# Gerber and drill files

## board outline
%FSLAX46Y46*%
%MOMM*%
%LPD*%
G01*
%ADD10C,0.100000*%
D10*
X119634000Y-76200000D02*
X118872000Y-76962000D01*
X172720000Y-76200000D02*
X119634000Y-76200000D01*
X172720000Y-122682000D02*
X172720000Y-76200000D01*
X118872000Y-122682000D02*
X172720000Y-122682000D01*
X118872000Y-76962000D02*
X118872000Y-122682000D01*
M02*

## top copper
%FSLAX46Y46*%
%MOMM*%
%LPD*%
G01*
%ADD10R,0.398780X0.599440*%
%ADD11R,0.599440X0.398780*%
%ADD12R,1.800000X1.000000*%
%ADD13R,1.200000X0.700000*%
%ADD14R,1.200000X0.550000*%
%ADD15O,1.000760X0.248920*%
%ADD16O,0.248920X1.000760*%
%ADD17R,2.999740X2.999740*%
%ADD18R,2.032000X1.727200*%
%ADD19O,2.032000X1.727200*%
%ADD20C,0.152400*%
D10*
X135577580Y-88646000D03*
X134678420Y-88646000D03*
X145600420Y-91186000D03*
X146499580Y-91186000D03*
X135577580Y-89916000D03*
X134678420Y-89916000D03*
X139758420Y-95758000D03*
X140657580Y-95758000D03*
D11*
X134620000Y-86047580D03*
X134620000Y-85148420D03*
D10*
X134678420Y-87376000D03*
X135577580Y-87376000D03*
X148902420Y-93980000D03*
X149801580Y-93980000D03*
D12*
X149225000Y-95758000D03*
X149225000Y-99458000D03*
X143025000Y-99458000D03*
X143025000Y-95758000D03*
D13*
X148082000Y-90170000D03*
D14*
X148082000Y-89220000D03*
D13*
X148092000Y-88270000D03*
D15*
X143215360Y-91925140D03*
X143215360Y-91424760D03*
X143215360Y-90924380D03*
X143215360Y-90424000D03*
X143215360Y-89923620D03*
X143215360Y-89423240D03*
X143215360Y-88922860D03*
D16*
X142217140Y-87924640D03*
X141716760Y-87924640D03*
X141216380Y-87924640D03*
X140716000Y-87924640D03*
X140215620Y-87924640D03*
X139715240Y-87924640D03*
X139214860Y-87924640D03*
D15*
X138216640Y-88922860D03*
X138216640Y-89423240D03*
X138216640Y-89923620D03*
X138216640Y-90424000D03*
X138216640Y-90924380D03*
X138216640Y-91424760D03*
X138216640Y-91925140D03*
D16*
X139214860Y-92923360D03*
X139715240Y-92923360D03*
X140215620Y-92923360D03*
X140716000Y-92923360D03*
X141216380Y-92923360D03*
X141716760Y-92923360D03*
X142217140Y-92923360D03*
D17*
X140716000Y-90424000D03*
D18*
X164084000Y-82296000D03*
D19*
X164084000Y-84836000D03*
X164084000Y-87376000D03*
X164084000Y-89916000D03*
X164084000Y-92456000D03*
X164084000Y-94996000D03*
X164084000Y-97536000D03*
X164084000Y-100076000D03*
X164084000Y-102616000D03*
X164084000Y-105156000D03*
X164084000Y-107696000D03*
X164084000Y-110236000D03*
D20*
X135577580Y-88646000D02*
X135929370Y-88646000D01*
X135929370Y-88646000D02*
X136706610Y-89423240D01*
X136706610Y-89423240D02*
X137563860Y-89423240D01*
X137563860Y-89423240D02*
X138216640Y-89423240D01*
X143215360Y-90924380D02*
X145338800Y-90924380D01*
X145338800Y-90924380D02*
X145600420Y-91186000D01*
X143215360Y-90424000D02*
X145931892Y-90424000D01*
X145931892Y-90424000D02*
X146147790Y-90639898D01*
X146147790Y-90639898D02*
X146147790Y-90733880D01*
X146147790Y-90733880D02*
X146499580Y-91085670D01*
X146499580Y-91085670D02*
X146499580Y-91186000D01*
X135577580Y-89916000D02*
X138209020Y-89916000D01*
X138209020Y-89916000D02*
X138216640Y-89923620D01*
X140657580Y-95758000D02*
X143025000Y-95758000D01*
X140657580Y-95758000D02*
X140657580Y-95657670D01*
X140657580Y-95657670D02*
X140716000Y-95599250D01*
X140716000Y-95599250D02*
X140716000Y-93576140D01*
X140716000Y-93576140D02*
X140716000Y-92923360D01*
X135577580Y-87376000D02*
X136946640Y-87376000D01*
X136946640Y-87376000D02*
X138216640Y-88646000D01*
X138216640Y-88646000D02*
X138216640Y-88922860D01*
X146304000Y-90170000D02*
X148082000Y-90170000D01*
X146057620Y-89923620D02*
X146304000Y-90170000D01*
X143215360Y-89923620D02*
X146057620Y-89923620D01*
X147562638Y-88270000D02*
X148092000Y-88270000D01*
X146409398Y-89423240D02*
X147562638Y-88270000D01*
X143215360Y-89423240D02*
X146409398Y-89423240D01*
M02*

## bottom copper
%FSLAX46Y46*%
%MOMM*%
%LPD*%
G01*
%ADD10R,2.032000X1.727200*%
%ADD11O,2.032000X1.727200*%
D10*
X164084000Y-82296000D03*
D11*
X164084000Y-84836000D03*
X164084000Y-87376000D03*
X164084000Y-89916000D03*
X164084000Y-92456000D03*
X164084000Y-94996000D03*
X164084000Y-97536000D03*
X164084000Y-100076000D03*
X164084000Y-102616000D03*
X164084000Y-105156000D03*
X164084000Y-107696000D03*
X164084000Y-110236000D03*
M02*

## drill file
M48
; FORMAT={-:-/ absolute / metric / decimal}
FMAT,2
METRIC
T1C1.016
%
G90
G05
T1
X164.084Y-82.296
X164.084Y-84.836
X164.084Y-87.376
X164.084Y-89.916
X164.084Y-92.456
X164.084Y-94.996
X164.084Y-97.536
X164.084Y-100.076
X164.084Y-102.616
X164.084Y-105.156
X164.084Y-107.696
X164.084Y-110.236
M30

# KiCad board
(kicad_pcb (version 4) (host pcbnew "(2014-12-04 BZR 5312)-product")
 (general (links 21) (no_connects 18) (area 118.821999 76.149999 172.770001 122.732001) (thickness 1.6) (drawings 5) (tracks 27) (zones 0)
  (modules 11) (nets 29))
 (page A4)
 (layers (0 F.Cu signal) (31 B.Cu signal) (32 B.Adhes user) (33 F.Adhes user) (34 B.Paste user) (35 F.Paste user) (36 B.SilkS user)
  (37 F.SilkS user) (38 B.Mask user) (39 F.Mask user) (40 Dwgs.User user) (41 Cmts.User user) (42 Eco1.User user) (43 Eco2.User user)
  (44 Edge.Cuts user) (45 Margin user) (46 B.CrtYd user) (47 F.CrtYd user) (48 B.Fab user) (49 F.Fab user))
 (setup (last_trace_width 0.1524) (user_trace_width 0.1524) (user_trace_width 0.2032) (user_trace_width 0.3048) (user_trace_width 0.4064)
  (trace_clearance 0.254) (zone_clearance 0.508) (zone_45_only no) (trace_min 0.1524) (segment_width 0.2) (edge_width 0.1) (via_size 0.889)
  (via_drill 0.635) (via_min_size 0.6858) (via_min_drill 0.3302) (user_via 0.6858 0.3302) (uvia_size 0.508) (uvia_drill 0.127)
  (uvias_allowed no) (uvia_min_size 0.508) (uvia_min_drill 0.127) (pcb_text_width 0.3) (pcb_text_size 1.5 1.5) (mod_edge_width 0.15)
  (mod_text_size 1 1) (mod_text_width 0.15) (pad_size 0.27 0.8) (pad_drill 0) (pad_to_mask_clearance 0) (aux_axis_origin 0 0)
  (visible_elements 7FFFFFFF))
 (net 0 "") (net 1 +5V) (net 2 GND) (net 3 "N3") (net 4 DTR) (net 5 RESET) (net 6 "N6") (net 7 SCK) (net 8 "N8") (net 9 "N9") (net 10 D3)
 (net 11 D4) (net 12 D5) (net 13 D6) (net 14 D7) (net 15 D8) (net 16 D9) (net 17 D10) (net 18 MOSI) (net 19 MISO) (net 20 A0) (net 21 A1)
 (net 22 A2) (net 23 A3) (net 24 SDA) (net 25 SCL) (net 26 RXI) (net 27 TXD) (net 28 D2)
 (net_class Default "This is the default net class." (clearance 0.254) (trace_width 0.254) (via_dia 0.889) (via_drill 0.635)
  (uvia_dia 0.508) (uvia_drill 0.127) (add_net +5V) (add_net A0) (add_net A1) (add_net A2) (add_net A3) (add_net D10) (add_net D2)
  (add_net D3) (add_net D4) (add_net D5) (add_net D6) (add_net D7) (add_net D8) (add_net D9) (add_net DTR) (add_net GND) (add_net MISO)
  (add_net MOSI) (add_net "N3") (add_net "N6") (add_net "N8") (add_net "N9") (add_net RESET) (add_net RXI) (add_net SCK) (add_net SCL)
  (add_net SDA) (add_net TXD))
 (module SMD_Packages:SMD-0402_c (layer F.Cu) (at 135.128 88.646 180)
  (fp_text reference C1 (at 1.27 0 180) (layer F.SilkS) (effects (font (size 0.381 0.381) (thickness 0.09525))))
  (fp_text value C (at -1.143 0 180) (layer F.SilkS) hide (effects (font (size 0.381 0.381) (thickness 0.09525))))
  (pad 1 smd rect (at -0.44958 0 180) (size 0.39878 0.59944) (layers F.Cu F.Paste F.Mask) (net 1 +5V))
  (pad 2 smd rect (at 0.44958 0 180) (size 0.39878 0.59944) (layers F.Cu F.Paste F.Mask) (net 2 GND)))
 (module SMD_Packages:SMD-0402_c (layer F.Cu) (at 146.05 91.186)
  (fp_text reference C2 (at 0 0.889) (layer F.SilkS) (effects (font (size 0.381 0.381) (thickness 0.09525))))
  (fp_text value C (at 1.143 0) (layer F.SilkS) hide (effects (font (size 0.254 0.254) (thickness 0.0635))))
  (pad 1 smd rect (at -0.44958 0) (size 0.39878 0.59944) (layers F.Cu F.Paste F.Mask) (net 1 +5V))
  (pad 2 smd rect (at 0.44958 0) (size 0.39878 0.59944) (layers F.Cu F.Paste F.Mask) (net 2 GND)))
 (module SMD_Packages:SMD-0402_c (layer F.Cu) (at 135.128 89.916 180)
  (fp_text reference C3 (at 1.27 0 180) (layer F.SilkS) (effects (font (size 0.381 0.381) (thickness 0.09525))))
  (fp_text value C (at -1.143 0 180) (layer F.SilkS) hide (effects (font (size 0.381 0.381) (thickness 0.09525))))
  (pad 1 smd rect (at -0.44958 0 180) (size 0.39878 0.59944) (layers F.Cu F.Paste F.Mask) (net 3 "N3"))
  (pad 2 smd rect (at 0.44958 0 180) (size 0.39878 0.59944) (layers F.Cu F.Paste F.Mask) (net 2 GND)))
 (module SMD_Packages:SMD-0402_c (layer F.Cu) (at 140.208 95.758)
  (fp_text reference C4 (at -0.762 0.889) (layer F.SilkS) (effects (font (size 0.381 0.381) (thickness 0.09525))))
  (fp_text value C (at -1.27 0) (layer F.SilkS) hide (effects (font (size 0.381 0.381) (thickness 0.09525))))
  (pad 1 smd rect (at -0.44958 0) (size 0.39878 0.59944) (layers F.Cu F.Paste F.Mask) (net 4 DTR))
  (pad 2 smd rect (at 0.44958 0) (size 0.39878 0.59944) (layers F.Cu F.Paste F.Mask) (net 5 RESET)))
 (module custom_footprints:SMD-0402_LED (layer F.Cu) (at 134.62 85.598 90)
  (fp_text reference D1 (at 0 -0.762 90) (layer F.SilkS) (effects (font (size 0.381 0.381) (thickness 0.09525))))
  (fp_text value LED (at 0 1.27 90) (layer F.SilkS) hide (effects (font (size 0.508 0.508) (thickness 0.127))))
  (pad 1 smd rect (at -0.44958 0 90) (size 0.39878 0.59944) (layers F.Cu F.Paste F.Mask) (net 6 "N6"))
  (pad 2 smd rect (at 0.44958 0 90) (size 0.39878 0.59944) (layers F.Cu F.Paste F.Mask) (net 2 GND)))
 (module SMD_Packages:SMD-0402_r (layer F.Cu) (at 135.128 87.376)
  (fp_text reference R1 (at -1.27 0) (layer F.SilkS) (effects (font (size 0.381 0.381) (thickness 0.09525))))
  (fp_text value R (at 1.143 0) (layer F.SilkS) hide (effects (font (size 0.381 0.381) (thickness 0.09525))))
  (pad 1 smd rect (at -0.44958 0) (size 0.39878 0.59944) (layers F.Cu F.Paste F.Mask) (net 6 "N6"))
  (pad 2 smd rect (at 0.44958 0) (size 0.39878 0.59944) (layers F.Cu F.Paste F.Mask) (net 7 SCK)))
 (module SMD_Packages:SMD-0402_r (layer F.Cu) (at 149.352 93.98)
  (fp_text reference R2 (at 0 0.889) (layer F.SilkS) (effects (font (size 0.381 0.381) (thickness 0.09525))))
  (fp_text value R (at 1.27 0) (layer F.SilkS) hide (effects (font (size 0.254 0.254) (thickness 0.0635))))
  (pad 1 smd rect (at -0.44958 0) (size 0.39878 0.59944) (layers F.Cu F.Paste F.Mask) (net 1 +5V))
  (pad 2 smd rect (at 0.44958 0) (size 0.39878 0.59944) (layers F.Cu F.Paste F.Mask) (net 5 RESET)))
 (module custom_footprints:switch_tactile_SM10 (layer F.Cu) (at 149.225 95.758 180) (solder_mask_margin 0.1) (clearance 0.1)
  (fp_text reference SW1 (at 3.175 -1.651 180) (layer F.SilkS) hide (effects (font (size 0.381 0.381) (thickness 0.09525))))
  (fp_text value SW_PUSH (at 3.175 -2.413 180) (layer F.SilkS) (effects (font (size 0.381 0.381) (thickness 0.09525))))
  (pad 1 smd rect (at 0 0 180) (size 1.8 1) (layers F.Cu F.Paste F.Mask) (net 5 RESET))
  (pad 2 smd rect (at 0 -3.7 180) (size 1.8 1) (layers F.Cu F.Paste F.Mask) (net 2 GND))
  (pad 2 smd rect (at 6.2 -3.7 180) (size 1.8 1) (layers F.Cu F.Paste F.Mask) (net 2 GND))
  (pad 1 smd rect (at 6.2 0 180) (size 1.8 1) (layers F.Cu F.Paste F.Mask) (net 5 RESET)))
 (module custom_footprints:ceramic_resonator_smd (layer F.Cu) (at 148.082 90.17 90) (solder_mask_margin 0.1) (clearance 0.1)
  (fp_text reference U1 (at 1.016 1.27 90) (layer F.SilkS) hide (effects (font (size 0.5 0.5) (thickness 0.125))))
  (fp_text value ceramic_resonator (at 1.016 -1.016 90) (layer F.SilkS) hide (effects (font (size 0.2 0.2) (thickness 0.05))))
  (pad 1 smd rect (at 0 0 90) (size 0.7 1.2) (layers F.Cu F.Paste F.Mask) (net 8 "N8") (solder_mask_margin 0.1) (clearance 0.1))
  (pad 3 smd rect (at 0.95 0 90) (size 0.55 1.2) (layers F.Cu F.Paste F.Mask) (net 2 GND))
  (pad 2 smd rect (at 1.9 0.01 90) (size 0.7 1.2) (layers F.Cu F.Paste F.Mask) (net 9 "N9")))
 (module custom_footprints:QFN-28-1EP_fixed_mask (layer F.Cu) (at 140.716 90.424 180) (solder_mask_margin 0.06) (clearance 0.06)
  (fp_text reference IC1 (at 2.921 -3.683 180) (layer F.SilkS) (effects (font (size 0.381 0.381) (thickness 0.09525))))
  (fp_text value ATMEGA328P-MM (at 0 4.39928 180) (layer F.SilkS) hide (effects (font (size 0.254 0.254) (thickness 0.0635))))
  (pad 1 smd oval (at -2.49936 -1.50114 180) (size 1.00076 0.24892) (layers F.Cu F.Paste F.Mask) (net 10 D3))
  (pad 2 smd oval (at -2.49936 -1.00076 180) (size 1.00076 0.24892) (layers F.Cu F.Paste F.Mask) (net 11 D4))
  (pad 3 smd oval (at -2.49936 -0.50038 180) (size 1.00076 0.24892) (layers F.Cu F.Paste F.Mask) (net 1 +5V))
  (pad 4 smd oval (at -2.49936 0 180) (size 1.00076 0.24892) (layers F.Cu F.Paste F.Mask) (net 2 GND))
  (pad 5 smd oval (at -2.49936 0.50038 180) (size 1.00076 0.24892) (layers F.Cu F.Paste F.Mask) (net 8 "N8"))
  (pad 6 smd oval (at -2.49936 1.00076 180) (size 1.00076 0.24892) (layers F.Cu F.Paste F.Mask) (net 9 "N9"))
  (pad 7 smd oval (at -2.49936 1.50114 180) (size 1.00076 0.24892) (layers F.Cu F.Paste F.Mask) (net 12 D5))
  (pad 8 smd oval (at -1.50114 2.49936 270) (size 1.00076 0.24892) (layers F.Cu F.Paste F.Mask) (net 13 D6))
  (pad 9 smd oval (at -1.00076 2.49936 270) (size 1.00076 0.24892) (layers F.Cu F.Paste F.Mask) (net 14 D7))
  (pad 10 smd oval (at -0.50038 2.49936 270) (size 1.00076 0.24892) (layers F.Cu F.Paste F.Mask) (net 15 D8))
  (pad 11 smd oval (at 0 2.49936 270) (size 1.00076 0.24892) (layers F.Cu F.Paste F.Mask) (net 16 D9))
  (pad 12 smd oval (at 0.50038 2.49936 270) (size 1.00076 0.24892) (layers F.Cu F.Paste F.Mask) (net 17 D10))
  (pad 13 smd oval (at 1.00076 2.49936 270) (size 1.00076 0.24892) (layers F.Cu F.Paste F.Mask) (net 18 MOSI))
  (pad 14 smd oval (at 1.50114 2.49936 270) (size 1.00076 0.24892) (layers F.Cu F.Paste F.Mask) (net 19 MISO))
  (pad 15 smd oval (at 2.49936 1.50114) (size 1.00076 0.24892) (layers F.Cu F.Paste F.Mask) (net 7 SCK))
  (pad 16 smd oval (at 2.49936 1.00076) (size 1.00076 0.24892) (layers F.Cu F.Paste F.Mask) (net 1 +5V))
  (pad 17 smd oval (at 2.49936 0.50038) (size 1.00076 0.24892) (layers F.Cu F.Paste F.Mask) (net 3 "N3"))
  (pad 18 smd oval (at 2.49936 0) (size 1.00076 0.24892) (layers F.Cu F.Paste F.Mask) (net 2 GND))
  (pad 19 smd oval (at 2.49936 -0.50038) (size 1.00076 0.24892) (layers F.Cu F.Paste F.Mask) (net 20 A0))
  (pad 20 smd oval (at 2.49936 -1.00076) (size 1.00076 0.24892) (layers F.Cu F.Paste F.Mask) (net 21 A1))
  (pad 21 smd oval (at 2.49936 -1.50114) (size 1.00076 0.24892) (layers F.Cu F.Paste F.Mask) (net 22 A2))
  (pad 22 smd oval (at 1.50114 -2.49936 90) (size 1.00076 0.24892) (layers F.Cu F.Paste F.Mask) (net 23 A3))
  (pad 23 smd oval (at 1.00076 -2.49936 90) (size 1.00076 0.24892) (layers F.Cu F.Paste F.Mask) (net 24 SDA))
  (pad 24 smd oval (at 0.50038 -2.49936 90) (size 1.00076 0.24892) (layers F.Cu F.Paste F.Mask) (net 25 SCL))
  (pad 25 smd oval (at 0 -2.49936 90) (size 1.00076 0.24892) (layers F.Cu F.Paste F.Mask) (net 5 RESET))
  (pad 26 smd oval (at -0.50038 -2.49936 90) (size 1.00076 0.24892) (layers F.Cu F.Paste F.Mask) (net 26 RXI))
  (pad 27 smd oval (at -1.00076 -2.49936 90) (size 1.00076 0.24892) (layers F.Cu F.Paste F.Mask) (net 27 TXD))
  (pad 28 smd oval (at -1.50114 -2.49936 90) (size 1.00076 0.24892) (layers F.Cu F.Paste F.Mask) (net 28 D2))
  (pad 29 smd rect (at 0 0 90) (size 2.99974 2.99974) (layers F.Cu)))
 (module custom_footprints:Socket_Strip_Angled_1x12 (layer F.Cu) (at 164.084 96.266 90)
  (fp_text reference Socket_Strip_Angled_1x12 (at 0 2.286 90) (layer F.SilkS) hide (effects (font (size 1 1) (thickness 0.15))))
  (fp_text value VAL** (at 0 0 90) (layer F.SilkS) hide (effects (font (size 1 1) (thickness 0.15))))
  (pad 1 thru_hole rect (at 13.97 0 270) (size 1.7272 2.032) (drill 1.016) (layers *.Cu *.Mask F.SilkS))
  (pad 2 thru_hole oval (at 11.43 0 270) (size 1.7272 2.032) (drill 1.016) (layers *.Cu *.Mask F.SilkS))
  (pad 3 thru_hole oval (at 8.89 0 270) (size 1.7272 2.032) (drill 1.016) (layers *.Cu *.Mask F.SilkS))
  (pad 4 thru_hole oval (at 6.35 0 270) (size 1.7272 2.032) (drill 1.016) (layers *.Cu *.Mask F.SilkS))
  (pad 5 thru_hole oval (at 3.81 0 270) (size 1.7272 2.032) (drill 1.016) (layers *.Cu *.Mask F.SilkS))
  (pad 6 thru_hole oval (at 1.27 0 270) (size 1.7272 2.032) (drill 1.016) (layers *.Cu *.Mask F.SilkS))
  (pad 7 thru_hole oval (at -1.27 0 270) (size 1.7272 2.032) (drill 1.016) (layers *.Cu *.Mask F.SilkS))
  (pad 8 thru_hole oval (at -3.81 0 270) (size 1.7272 2.032) (drill 1.016) (layers *.Cu *.Mask F.SilkS))
  (pad 9 thru_hole oval (at -6.35 0 270) (size 1.7272 2.032) (drill 1.016) (layers *.Cu *.Mask F.SilkS))
  (pad 10 thru_hole oval (at -8.89 0 270) (size 1.7272 2.032) (drill 1.016) (layers *.Cu *.Mask F.SilkS))
  (pad 11 thru_hole oval (at -11.43 0 270) (size 1.7272 2.032) (drill 1.016) (layers *.Cu *.Mask F.SilkS))
  (pad 12 thru_hole oval (at -13.97 0 270) (size 1.7272 2.032) (drill 1.016) (layers *.Cu *.Mask F.SilkS)))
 (gr_line (start 119.634 76.2) (end 118.872 76.962) (angle 90) (layer Edge.Cuts) (width 0.1))
 (gr_line (start 172.72 76.2) (end 119.634 76.2) (angle 90) (layer Edge.Cuts) (width 0.1))
 (gr_line (start 172.72 122.682) (end 172.72 76.2) (angle 90) (layer Edge.Cuts) (width 0.1))
 (gr_line (start 118.872 122.682) (end 172.72 122.682) (angle 90) (layer Edge.Cuts) (width 0.1))
 (gr_line (start 118.872 76.962) (end 118.872 122.682) (angle 90) (layer Edge.Cuts) (width 0.1))
 (segment (start 135.57758 88.646) (end 135.92937 88.646) (width 0.1524) (layer F.Cu) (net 1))
 (segment (start 135.92937 88.646) (end 136.70661 89.42324) (width 0.1524) (layer F.Cu) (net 1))
 (segment (start 136.70661 89.42324) (end 137.56386 89.42324) (width 0.1524) (layer F.Cu) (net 1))
 (segment (start 137.56386 89.42324) (end 138.21664 89.42324) (width 0.1524) (layer F.Cu) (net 1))
 (segment (start 143.21536 90.92438) (end 145.3388 90.92438) (width 0.1524) (layer F.Cu) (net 1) (status 400000))
 (segment (start 145.3388 90.92438) (end 145.60042 91.186) (width 0.1524) (layer F.Cu) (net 1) (status 800000))
 (segment (start 143.21536 90.424) (end 145.931892 90.424) (width 0.1524) (layer F.Cu) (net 2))
 (segment (start 145.931892 90.424) (end 146.14779 90.639898) (width 0.1524) (layer F.Cu) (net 2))
 (segment (start 146.14779 90.639898) (end 146.14779 90.73388) (width 0.1524) (layer F.Cu) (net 2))
 (segment (start 146.14779 90.73388) (end 146.49958 91.08567) (width 0.1524) (layer F.Cu) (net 2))
 (segment (start 146.49958 91.08567) (end 146.49958 91.186) (width 0.1524) (layer F.Cu) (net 2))
 (segment (start 135.57758 89.916) (end 138.20902 89.916) (width 0.1524) (layer F.Cu) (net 3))
 (segment (start 138.20902 89.916) (end 138.21664 89.92362) (width 0.1524) (layer F.Cu) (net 3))
 (segment (start 140.65758 95.758) (end 143.025 95.758) (width 0.1524) (layer F.Cu) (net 5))
 (segment (start 140.65758 95.758) (end 140.65758 95.65767) (width 0.1524) (layer F.Cu) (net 5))
 (segment (start 140.65758 95.65767) (end 140.716 95.59925) (width 0.1524) (layer F.Cu) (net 5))
 (segment (start 140.716 95.59925) (end 140.716 93.57614) (width 0.1524) (layer F.Cu) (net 5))
 (segment (start 140.716 93.57614) (end 140.716 92.92336) (width 0.1524) (layer F.Cu) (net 5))
 (segment (start 135.57758 87.376) (end 136.94664 87.376) (width 0.1524) (layer F.Cu) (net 7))
 (segment (start 136.94664 87.376) (end 138.21664 88.646) (width 0.1524) (layer F.Cu) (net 7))
 (segment (start 138.21664 88.646) (end 138.21664 88.92286) (width 0.1524) (layer F.Cu) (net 7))
 (segment (start 146.304 90.17) (end 148.082 90.17) (width 0.1524) (layer F.Cu) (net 8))
 (segment (start 146.05762 89.92362) (end 146.304 90.17) (width 0.1524) (layer F.Cu) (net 8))
 (segment (start 143.21536 89.92362) (end 146.05762 89.92362) (width 0.1524) (layer F.Cu) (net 8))
 (segment (start 147.562638 88.27) (end 148.092 88.27) (width 0.1524) (layer F.Cu) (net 9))
 (segment (start 146.409398 89.42324) (end 147.562638 88.27) (width 0.1524) (layer F.Cu) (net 9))
 (segment (start 143.21536 89.42324) (end 146.409398 89.42324) (width 0.1524) (layer F.Cu) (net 9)))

